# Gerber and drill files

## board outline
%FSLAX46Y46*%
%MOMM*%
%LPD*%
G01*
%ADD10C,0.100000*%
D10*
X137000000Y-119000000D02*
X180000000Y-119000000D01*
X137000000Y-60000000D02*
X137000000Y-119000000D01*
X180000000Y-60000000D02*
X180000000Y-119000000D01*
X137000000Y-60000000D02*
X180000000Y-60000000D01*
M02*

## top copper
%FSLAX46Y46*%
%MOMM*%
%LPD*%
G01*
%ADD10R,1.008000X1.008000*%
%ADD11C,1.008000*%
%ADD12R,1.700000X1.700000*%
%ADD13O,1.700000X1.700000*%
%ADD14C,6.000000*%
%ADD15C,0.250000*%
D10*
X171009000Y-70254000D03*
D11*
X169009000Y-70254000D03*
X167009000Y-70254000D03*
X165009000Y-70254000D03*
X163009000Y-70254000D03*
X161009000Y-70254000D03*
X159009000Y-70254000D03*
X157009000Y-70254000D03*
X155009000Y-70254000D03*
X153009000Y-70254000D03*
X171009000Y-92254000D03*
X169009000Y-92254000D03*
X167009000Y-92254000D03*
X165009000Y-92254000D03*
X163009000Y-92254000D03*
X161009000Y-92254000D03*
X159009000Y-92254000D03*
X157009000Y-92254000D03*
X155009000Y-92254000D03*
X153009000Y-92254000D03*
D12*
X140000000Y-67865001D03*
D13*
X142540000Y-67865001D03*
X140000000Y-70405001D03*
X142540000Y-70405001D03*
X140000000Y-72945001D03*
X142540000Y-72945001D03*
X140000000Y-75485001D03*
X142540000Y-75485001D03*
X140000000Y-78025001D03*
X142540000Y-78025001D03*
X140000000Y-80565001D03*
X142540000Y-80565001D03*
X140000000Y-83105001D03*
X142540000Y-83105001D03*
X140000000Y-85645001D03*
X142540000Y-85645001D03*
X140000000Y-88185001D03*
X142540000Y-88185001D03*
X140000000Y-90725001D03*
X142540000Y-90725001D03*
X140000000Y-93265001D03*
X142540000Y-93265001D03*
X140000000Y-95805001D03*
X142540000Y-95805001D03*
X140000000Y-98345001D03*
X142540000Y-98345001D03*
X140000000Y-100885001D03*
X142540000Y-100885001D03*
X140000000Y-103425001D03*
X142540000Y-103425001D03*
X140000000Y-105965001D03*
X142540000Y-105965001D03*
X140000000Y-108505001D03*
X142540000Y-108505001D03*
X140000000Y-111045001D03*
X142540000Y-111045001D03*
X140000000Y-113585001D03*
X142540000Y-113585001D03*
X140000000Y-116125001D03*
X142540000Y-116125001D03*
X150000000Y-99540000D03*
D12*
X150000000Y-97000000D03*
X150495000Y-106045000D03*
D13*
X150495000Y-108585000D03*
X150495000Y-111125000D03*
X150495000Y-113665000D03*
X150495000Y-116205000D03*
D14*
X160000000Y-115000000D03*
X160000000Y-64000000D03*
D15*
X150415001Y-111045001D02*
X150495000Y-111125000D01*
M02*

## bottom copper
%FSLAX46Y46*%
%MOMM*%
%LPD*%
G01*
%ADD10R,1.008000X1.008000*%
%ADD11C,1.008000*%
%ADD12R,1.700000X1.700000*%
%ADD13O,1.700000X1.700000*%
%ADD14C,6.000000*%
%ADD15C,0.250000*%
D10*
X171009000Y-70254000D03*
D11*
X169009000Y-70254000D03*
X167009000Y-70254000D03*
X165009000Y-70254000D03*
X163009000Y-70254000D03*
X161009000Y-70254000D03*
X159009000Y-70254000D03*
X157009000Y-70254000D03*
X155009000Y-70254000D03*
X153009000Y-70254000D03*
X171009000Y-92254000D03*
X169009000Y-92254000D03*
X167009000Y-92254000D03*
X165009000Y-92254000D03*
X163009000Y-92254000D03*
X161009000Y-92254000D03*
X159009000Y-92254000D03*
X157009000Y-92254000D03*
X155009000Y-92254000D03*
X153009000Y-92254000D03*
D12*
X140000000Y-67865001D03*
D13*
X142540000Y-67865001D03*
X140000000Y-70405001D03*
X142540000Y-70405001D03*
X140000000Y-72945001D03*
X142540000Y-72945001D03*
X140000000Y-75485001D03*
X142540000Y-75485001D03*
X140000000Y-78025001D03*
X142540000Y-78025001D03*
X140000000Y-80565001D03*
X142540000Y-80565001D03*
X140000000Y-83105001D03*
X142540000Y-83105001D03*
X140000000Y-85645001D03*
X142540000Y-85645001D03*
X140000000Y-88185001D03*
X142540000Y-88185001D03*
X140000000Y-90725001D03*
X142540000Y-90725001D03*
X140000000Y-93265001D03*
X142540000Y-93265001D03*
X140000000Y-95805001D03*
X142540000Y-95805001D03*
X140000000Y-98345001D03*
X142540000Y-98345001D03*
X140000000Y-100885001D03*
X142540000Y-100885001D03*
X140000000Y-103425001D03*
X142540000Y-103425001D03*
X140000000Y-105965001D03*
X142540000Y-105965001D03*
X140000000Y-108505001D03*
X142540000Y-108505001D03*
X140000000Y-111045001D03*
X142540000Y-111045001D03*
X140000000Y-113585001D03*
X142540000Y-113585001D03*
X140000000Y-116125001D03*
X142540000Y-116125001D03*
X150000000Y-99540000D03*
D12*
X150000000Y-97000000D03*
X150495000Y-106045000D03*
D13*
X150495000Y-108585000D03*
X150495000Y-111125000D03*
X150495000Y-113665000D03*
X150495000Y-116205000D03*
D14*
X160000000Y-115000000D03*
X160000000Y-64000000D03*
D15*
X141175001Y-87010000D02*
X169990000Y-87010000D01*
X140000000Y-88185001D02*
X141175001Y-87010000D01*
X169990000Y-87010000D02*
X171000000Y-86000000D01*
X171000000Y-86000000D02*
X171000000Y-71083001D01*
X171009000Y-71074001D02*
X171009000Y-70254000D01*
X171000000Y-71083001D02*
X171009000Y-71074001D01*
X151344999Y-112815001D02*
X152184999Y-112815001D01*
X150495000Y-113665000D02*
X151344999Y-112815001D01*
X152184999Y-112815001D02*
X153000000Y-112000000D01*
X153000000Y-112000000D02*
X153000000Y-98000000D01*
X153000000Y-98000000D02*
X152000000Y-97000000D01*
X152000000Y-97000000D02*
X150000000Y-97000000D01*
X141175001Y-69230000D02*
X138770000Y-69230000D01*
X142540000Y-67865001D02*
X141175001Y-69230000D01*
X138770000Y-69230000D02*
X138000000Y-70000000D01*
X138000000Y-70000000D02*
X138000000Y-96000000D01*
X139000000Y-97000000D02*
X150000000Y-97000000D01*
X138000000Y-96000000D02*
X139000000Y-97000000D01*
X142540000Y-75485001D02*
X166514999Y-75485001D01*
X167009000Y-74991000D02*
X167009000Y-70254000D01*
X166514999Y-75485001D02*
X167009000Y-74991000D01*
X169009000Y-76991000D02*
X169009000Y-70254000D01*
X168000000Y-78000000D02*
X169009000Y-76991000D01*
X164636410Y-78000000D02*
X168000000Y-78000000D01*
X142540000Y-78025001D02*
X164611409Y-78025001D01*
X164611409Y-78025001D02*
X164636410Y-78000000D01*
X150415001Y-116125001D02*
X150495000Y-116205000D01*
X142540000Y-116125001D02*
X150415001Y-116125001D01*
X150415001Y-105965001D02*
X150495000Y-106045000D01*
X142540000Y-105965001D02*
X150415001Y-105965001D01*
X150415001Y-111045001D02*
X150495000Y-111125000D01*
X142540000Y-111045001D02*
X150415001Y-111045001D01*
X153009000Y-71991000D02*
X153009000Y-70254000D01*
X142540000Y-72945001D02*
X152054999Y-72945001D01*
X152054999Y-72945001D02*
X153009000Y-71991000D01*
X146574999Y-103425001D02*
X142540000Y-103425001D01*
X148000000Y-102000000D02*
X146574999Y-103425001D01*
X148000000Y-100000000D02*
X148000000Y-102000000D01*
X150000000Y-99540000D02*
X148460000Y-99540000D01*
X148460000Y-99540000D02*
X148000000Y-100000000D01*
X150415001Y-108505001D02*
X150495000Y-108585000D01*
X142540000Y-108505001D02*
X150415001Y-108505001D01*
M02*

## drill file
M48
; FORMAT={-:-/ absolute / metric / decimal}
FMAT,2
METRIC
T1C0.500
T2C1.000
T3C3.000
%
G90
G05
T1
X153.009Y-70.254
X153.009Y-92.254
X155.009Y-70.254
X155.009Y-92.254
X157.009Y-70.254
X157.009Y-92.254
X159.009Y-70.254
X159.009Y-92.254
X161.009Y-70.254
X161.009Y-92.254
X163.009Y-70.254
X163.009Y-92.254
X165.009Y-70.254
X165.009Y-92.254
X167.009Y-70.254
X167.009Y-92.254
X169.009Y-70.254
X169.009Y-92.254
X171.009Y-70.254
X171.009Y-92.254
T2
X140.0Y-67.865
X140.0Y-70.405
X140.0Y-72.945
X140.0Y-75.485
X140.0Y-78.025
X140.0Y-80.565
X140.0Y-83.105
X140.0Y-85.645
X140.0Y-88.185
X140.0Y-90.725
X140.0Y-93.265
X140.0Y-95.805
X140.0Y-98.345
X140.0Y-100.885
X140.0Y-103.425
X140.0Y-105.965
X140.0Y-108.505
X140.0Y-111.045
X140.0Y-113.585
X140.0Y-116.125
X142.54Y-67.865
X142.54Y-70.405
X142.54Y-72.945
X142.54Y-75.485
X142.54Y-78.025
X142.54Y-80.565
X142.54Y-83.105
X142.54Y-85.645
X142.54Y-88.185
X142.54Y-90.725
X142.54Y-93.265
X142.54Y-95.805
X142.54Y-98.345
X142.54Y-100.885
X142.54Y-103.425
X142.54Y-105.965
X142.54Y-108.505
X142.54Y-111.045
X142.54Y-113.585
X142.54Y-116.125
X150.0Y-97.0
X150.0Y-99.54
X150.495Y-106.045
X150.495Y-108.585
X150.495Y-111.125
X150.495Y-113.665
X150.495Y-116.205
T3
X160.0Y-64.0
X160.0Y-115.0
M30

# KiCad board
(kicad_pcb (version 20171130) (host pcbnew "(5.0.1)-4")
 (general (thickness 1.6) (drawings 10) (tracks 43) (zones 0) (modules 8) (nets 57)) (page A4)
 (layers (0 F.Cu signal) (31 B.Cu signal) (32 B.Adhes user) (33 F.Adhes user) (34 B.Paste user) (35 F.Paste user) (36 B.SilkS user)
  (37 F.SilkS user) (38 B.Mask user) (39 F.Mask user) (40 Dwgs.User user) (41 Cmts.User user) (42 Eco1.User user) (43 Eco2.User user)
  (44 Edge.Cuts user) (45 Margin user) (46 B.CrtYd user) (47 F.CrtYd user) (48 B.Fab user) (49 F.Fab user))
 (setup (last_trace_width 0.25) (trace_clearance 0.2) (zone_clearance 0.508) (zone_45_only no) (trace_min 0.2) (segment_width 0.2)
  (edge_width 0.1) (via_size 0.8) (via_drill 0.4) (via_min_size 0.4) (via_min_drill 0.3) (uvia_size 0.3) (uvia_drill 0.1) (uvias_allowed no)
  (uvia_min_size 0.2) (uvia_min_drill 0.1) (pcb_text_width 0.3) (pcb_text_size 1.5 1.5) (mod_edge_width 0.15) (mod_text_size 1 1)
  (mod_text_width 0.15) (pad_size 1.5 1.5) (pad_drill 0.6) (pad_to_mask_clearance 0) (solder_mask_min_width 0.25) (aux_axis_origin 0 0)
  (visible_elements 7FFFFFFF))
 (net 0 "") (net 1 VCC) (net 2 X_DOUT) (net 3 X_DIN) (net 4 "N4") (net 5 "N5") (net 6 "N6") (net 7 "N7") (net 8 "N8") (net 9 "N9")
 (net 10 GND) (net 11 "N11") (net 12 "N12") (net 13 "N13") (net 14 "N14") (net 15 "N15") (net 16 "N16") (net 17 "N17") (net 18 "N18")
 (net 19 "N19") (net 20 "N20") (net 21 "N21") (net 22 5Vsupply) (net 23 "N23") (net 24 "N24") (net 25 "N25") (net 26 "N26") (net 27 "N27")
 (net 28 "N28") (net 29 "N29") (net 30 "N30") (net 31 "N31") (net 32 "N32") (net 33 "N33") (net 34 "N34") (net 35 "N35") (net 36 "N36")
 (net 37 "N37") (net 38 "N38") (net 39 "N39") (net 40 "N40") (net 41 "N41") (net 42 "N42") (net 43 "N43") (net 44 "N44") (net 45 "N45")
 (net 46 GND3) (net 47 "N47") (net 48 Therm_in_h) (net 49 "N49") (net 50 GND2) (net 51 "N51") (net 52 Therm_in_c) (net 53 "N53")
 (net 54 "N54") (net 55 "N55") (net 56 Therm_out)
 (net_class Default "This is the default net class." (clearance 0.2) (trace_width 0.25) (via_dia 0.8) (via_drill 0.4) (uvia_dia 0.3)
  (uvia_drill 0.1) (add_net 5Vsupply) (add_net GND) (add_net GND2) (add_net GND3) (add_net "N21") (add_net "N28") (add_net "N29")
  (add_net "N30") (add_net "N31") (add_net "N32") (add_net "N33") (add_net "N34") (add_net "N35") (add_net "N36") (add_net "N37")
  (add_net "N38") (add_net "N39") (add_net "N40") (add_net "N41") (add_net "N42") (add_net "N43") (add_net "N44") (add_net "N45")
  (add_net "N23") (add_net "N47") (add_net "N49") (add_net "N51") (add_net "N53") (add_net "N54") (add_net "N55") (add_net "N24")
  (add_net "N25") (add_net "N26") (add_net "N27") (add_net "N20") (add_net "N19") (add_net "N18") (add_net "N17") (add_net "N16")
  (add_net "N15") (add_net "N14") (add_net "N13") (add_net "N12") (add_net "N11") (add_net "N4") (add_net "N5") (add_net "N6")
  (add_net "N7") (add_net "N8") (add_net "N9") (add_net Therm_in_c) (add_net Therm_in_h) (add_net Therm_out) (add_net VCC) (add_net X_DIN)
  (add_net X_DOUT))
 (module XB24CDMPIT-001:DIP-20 (layer F.Cu) (at 145 69 270)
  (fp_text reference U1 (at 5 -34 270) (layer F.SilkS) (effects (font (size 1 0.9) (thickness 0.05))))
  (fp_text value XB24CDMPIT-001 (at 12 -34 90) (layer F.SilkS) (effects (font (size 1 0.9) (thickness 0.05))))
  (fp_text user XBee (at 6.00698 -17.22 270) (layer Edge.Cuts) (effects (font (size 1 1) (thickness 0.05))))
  (pad 1 thru_hole rect (at 1.254 -26.009 270) (size 1.008 1.008) (drill 0.5) (layers *.Cu *.Mask) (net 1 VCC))
  (pad 2 thru_hole circle (at 1.254 -24.009 270) (size 1.008 1.008) (drill 0.5) (layers *.Cu *.Mask) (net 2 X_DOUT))
  (pad 3 thru_hole circle (at 1.254 -22.009 270) (size 1.008 1.008) (drill 0.5) (layers *.Cu *.Mask) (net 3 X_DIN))
  (pad 4 thru_hole circle (at 1.254 -20.009 270) (size 1.008 1.008) (drill 0.5) (layers *.Cu *.Mask) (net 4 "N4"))
  (pad 5 thru_hole circle (at 1.254 -18.009 270) (size 1.008 1.008) (drill 0.5) (layers *.Cu *.Mask) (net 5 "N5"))
  (pad 6 thru_hole circle (at 1.254 -16.009 270) (size 1.008 1.008) (drill 0.5) (layers *.Cu *.Mask) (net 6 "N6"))
  (pad 7 thru_hole circle (at 1.254 -14.009 270) (size 1.008 1.008) (drill 0.5) (layers *.Cu *.Mask) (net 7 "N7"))
  (pad 8 thru_hole circle (at 1.254 -12.009 270) (size 1.008 1.008) (drill 0.5) (layers *.Cu *.Mask) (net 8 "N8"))
  (pad 9 thru_hole circle (at 1.254 -10.009 270) (size 1.008 1.008) (drill 0.5) (layers *.Cu *.Mask) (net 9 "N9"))
  (pad 10 thru_hole circle (at 1.254 -8.009 270) (size 1.008 1.008) (drill 0.5) (layers *.Cu *.Mask) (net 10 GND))
  (pad 20 thru_hole circle (at 23.254 -26.009 270) (size 1.008 1.008) (drill 0.5) (layers *.Cu *.Mask) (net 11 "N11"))
  (pad 19 thru_hole circle (at 23.254 -24.009 270) (size 1.008 1.008) (drill 0.5) (layers *.Cu *.Mask) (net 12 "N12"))
  (pad 18 thru_hole circle (at 23.254 -22.009 270) (size 1.008 1.008) (drill 0.5) (layers *.Cu *.Mask) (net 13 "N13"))
  (pad 17 thru_hole circle (at 23.254 -20.009 270) (size 1.008 1.008) (drill 0.5) (layers *.Cu *.Mask) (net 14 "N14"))
  (pad 16 thru_hole circle (at 23.254 -18.009 270) (size 1.008 1.008) (drill 0.5) (layers *.Cu *.Mask) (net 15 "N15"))
  (pad 15 thru_hole circle (at 23.254 -16.009 270) (size 1.008 1.008) (drill 0.5) (layers *.Cu *.Mask) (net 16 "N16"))
  (pad 14 thru_hole circle (at 23.254 -14.009 270) (size 1.008 1.008) (drill 0.5) (layers *.Cu *.Mask) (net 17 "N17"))
  (pad 13 thru_hole circle (at 23.254 -12.009 270) (size 1.008 1.008) (drill 0.5) (layers *.Cu *.Mask) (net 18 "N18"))
  (pad 12 thru_hole circle (at 23.254 -10.009 270) (size 1.008 1.008) (drill 0.5) (layers *.Cu *.Mask) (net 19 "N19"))
  (pad 11 thru_hole circle (at 23.254 -8.009 270) (size 1.008 1.008) (drill 0.5) (layers *.Cu *.Mask) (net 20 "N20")))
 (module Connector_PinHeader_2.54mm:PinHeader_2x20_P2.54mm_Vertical (layer F.Cu) (at 140 67.865001)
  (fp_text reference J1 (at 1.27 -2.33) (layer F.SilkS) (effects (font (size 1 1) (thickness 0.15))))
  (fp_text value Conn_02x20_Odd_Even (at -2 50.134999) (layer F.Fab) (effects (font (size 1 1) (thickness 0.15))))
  (pad 1 thru_hole rect (at 0 0) (size 1.7 1.7) (drill 1) (layers *.Cu *.Mask) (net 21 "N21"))
  (pad 2 thru_hole oval (at 2.54 0) (size 1.7 1.7) (drill 1) (layers *.Cu *.Mask) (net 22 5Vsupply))
  (pad 3 thru_hole oval (at 0 2.54) (size 1.7 1.7) (drill 1) (layers *.Cu *.Mask) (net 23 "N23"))
  (pad 4 thru_hole oval (at 2.54 2.54) (size 1.7 1.7) (drill 1) (layers *.Cu *.Mask) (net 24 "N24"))
  (pad 5 thru_hole oval (at 0 5.08) (size 1.7 1.7) (drill 1) (layers *.Cu *.Mask) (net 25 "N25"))
  (pad 6 thru_hole oval (at 2.54 5.08) (size 1.7 1.7) (drill 1) (layers *.Cu *.Mask) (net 10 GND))
  (pad 7 thru_hole oval (at 0 7.62) (size 1.7 1.7) (drill 1) (layers *.Cu *.Mask) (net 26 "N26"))
  (pad 8 thru_hole oval (at 2.54 7.62) (size 1.7 1.7) (drill 1) (layers *.Cu *.Mask) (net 3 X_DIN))
  (pad 9 thru_hole oval (at 0 10.16) (size 1.7 1.7) (drill 1) (layers *.Cu *.Mask) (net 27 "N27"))
  (pad 10 thru_hole oval (at 2.54 10.16) (size 1.7 1.7) (drill 1) (layers *.Cu *.Mask) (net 2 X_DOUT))
  (pad 11 thru_hole oval (at 0 12.7) (size 1.7 1.7) (drill 1) (layers *.Cu *.Mask) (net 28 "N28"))
  (pad 12 thru_hole oval (at 2.54 12.7) (size 1.7 1.7) (drill 1) (layers *.Cu *.Mask) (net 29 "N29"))
  (pad 13 thru_hole oval (at 0 15.24) (size 1.7 1.7) (drill 1) (layers *.Cu *.Mask) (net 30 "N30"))
  (pad 14 thru_hole oval (at 2.54 15.24) (size 1.7 1.7) (drill 1) (layers *.Cu *.Mask) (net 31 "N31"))
  (pad 15 thru_hole oval (at 0 17.78) (size 1.7 1.7) (drill 1) (layers *.Cu *.Mask) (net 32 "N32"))
  (pad 16 thru_hole oval (at 2.54 17.78) (size 1.7 1.7) (drill 1) (layers *.Cu *.Mask) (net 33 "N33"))
  (pad 17 thru_hole oval (at 0 20.32) (size 1.7 1.7) (drill 1) (layers *.Cu *.Mask) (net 1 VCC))
  (pad 18 thru_hole oval (at 2.54 20.32) (size 1.7 1.7) (drill 1) (layers *.Cu *.Mask) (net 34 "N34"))
  (pad 19 thru_hole oval (at 0 22.86) (size 1.7 1.7) (drill 1) (layers *.Cu *.Mask) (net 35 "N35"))
  (pad 20 thru_hole oval (at 2.54 22.86) (size 1.7 1.7) (drill 1) (layers *.Cu *.Mask) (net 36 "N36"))
  (pad 21 thru_hole oval (at 0 25.4) (size 1.7 1.7) (drill 1) (layers *.Cu *.Mask) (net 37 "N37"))
  (pad 22 thru_hole oval (at 2.54 25.4) (size 1.7 1.7) (drill 1) (layers *.Cu *.Mask) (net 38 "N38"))
  (pad 23 thru_hole oval (at 0 27.94) (size 1.7 1.7) (drill 1) (layers *.Cu *.Mask) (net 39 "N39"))
  (pad 24 thru_hole oval (at 2.54 27.94) (size 1.7 1.7) (drill 1) (layers *.Cu *.Mask) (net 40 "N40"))
  (pad 25 thru_hole oval (at 0 30.48) (size 1.7 1.7) (drill 1) (layers *.Cu *.Mask) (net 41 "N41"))
  (pad 26 thru_hole oval (at 2.54 30.48) (size 1.7 1.7) (drill 1) (layers *.Cu *.Mask) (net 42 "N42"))
  (pad 27 thru_hole oval (at 0 33.02) (size 1.7 1.7) (drill 1) (layers *.Cu *.Mask) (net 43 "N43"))
  (pad 28 thru_hole oval (at 2.54 33.02) (size 1.7 1.7) (drill 1) (layers *.Cu *.Mask) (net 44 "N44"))
  (pad 29 thru_hole oval (at 0 35.56) (size 1.7 1.7) (drill 1) (layers *.Cu *.Mask) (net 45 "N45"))
  (pad 30 thru_hole oval (at 2.54 35.56) (size 1.7 1.7) (drill 1) (layers *.Cu *.Mask) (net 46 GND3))
  (pad 31 thru_hole oval (at 0 38.1) (size 1.7 1.7) (drill 1) (layers *.Cu *.Mask) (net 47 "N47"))
  (pad 32 thru_hole oval (at 2.54 38.1) (size 1.7 1.7) (drill 1) (layers *.Cu *.Mask) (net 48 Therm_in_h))
  (pad 33 thru_hole oval (at 0 40.64) (size 1.7 1.7) (drill 1) (layers *.Cu *.Mask) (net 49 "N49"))
  (pad 34 thru_hole oval (at 2.54 40.64) (size 1.7 1.7) (drill 1) (layers *.Cu *.Mask) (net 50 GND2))
  (pad 35 thru_hole oval (at 0 43.18) (size 1.7 1.7) (drill 1) (layers *.Cu *.Mask) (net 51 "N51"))
  (pad 36 thru_hole oval (at 2.54 43.18) (size 1.7 1.7) (drill 1) (layers *.Cu *.Mask) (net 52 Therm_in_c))
  (pad 37 thru_hole oval (at 0 45.72) (size 1.7 1.7) (drill 1) (layers *.Cu *.Mask) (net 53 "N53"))
  (pad 38 thru_hole oval (at 2.54 45.72) (size 1.7 1.7) (drill 1) (layers *.Cu *.Mask) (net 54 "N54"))
  (pad 39 thru_hole oval (at 0 48.26) (size 1.7 1.7) (drill 1) (layers *.Cu *.Mask) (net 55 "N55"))
  (pad 40 thru_hole oval (at 2.54 48.26) (size 1.7 1.7) (drill 1) (layers *.Cu *.Mask) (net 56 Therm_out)))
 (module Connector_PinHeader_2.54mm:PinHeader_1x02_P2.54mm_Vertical (layer F.Cu) (at 150 97)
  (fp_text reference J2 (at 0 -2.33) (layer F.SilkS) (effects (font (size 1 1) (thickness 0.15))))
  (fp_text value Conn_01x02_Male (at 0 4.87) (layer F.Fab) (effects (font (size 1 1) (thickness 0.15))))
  (pad 2 thru_hole oval (at 0 2.54) (size 1.7 1.7) (drill 1) (layers *.Cu *.Mask) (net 46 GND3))
  (pad 1 thru_hole rect (at 0 0) (size 1.7 1.7) (drill 1) (layers *.Cu *.Mask) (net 22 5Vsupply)))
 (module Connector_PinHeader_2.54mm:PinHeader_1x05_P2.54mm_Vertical (layer F.Cu) (at 150.495 106.045)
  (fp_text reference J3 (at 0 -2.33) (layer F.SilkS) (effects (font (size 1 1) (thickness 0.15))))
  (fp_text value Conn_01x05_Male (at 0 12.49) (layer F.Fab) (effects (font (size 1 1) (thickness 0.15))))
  (pad 1 thru_hole rect (at 0 0) (size 1.7 1.7) (drill 1) (layers *.Cu *.Mask) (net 48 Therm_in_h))
  (pad 2 thru_hole oval (at 0 2.54) (size 1.7 1.7) (drill 1) (layers *.Cu *.Mask) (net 50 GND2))
  (pad 3 thru_hole oval (at 0 5.08) (size 1.7 1.7) (drill 1) (layers *.Cu *.Mask) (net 52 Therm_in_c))
  (pad 4 thru_hole oval (at 0 7.62) (size 1.7 1.7) (drill 1) (layers *.Cu *.Mask) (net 22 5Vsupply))
  (pad 5 thru_hole oval (at 0 10.16) (size 1.7 1.7) (drill 1) (layers *.Cu *.Mask) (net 56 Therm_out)))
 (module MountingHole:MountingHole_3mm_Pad (layer F.Cu) (at 160 115)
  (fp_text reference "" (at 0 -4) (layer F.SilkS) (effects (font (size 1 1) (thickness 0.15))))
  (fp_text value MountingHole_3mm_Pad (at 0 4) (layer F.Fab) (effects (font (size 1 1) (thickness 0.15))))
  (pad 1 thru_hole circle (at 0 0) (size 6 6) (drill 3) (layers *.Cu *.Mask)))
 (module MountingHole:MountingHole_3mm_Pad (layer F.Cu) (at 160 64)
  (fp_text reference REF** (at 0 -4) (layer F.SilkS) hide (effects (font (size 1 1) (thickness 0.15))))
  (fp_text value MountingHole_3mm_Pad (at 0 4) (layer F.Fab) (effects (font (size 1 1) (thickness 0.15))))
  (pad 1 thru_hole circle (at 0 0) (size 6 6) (drill 3) (layers *.Cu *.Mask)))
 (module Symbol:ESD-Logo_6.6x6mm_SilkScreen (layer F.Cu) (at 175 114)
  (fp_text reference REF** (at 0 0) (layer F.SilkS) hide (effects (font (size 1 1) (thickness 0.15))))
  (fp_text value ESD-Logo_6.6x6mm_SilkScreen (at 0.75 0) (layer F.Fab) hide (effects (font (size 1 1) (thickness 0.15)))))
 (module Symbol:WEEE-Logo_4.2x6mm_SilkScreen (layer F.Cu) (at 168 114)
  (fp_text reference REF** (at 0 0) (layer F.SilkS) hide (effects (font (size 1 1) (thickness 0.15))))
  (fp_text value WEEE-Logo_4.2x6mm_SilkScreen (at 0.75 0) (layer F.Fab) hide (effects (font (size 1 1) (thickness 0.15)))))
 (gr_line (start 137 119) (end 180 119) (layer Edge.Cuts) (width 0.1))
 (gr_line (start 137 60) (end 137 119) (layer Edge.Cuts) (width 0.1))
 (gr_line (start 180 60) (end 180 119) (layer Edge.Cuts) (width 0.1))
 (gr_line (start 137 60) (end 180 60) (layer Edge.Cuts) (width 0.1))
 (segment (start 141.175001 87.01) (end 169.99 87.01) (width 0.25) (layer B.Cu) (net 1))
 (segment (start 140 88.185001) (end 141.175001 87.01) (width 0.25) (layer B.Cu) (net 1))
 (segment (start 169.99 87.01) (end 171 86) (width 0.25) (layer B.Cu) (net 1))
 (segment (start 171 86) (end 171 71.083001) (width 0.25) (layer B.Cu) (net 1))
 (segment (start 171.009 71.074001) (end 171.009 70.254) (width 0.25) (layer B.Cu) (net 1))
 (segment (start 171 71.083001) (end 171.009 71.074001) (width 0.25) (layer B.Cu) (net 1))
 (segment (start 151.344999 112.815001) (end 152.184999 112.815001) (width 0.25) (layer B.Cu) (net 22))
 (segment (start 150.495 113.665) (end 151.344999 112.815001) (width 0.25) (layer B.Cu) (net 22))
 (segment (start 152.184999 112.815001) (end 153 112) (width 0.25) (layer B.Cu) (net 22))
 (segment (start 153 112) (end 153 98) (width 0.25) (layer B.Cu) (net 22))
 (segment (start 153 98) (end 152 97) (width 0.25) (layer B.Cu) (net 22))
 (segment (start 152 97) (end 150 97) (width 0.25) (layer B.Cu) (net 22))
 (segment (start 141.175001 69.23) (end 138.77 69.23) (width 0.25) (layer B.Cu) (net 22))
 (segment (start 142.54 67.865001) (end 141.175001 69.23) (width 0.25) (layer B.Cu) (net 22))
 (segment (start 138.77 69.23) (end 138 70) (width 0.25) (layer B.Cu) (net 22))
 (segment (start 138 70) (end 138 96) (width 0.25) (layer B.Cu) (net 22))
 (segment (start 139 97) (end 150 97) (width 0.25) (layer B.Cu) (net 22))
 (segment (start 138 96) (end 139 97) (width 0.25) (layer B.Cu) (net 22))
 (segment (start 142.54 75.485001) (end 166.514999 75.485001) (width 0.25) (layer B.Cu) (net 3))
 (segment (start 167.009 74.991) (end 167.009 70.254) (width 0.25) (layer B.Cu) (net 3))
 (segment (start 166.514999 75.485001) (end 167.009 74.991) (width 0.25) (layer B.Cu) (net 3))
 (segment (start 169.009 76.991) (end 169.009 70.254) (width 0.25) (layer B.Cu) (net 2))
 (segment (start 168 78) (end 169.009 76.991) (width 0.25) (layer B.Cu) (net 2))
 (segment (start 164.63641 78) (end 168 78) (width 0.25) (layer B.Cu) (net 2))
 (segment (start 142.54 78.025001) (end 164.611409 78.025001) (width 0.25) (layer B.Cu) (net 2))
 (segment (start 164.611409 78.025001) (end 164.63641 78) (width 0.25) (layer B.Cu) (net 2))
 (segment (start 150.415001 116.125001) (end 150.495 116.205) (width 0.25) (layer B.Cu) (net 56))
 (segment (start 142.54 116.125001) (end 150.415001 116.125001) (width 0.25) (layer B.Cu) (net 56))
 (segment (start 150.415001 105.965001) (end 150.495 106.045) (width 0.25) (layer B.Cu) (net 48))
 (segment (start 142.54 105.965001) (end 150.415001 105.965001) (width 0.25) (layer B.Cu) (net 48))
 (segment (start 150.415001 111.045001) (end 150.495 111.125) (width 0.25) (layer F.Cu) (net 52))
 (segment (start 150.415001 111.045001) (end 150.495 111.125) (width 0.25) (layer B.Cu) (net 52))
 (segment (start 142.54 111.045001) (end 150.415001 111.045001) (width 0.25) (layer B.Cu) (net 52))
 (segment (start 153.009 71.991) (end 153.009 70.254) (width 0.25) (layer B.Cu) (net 10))
 (segment (start 142.54 72.945001) (end 152.054999 72.945001) (width 0.25) (layer B.Cu) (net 10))
 (segment (start 152.054999 72.945001) (end 153.009 71.991) (width 0.25) (layer B.Cu) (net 10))
 (segment (start 146.574999 103.425001) (end 142.54 103.425001) (width 0.25) (layer B.Cu) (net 46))
 (segment (start 148 102) (end 146.574999 103.425001) (width 0.25) (layer B.Cu) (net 46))
 (segment (start 148 100) (end 148 102) (width 0.25) (layer B.Cu) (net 46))
 (segment (start 150 99.54) (end 148.46 99.54) (width 0.25) (layer B.Cu) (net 46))
 (segment (start 148.46 99.54) (end 148 100) (width 0.25) (layer B.Cu) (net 46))
 (segment (start 150.415001 108.505001) (end 150.495 108.585) (width 0.25) (layer B.Cu) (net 50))
 (segment (start 142.54 108.505001) (end 150.415001 108.505001) (width 0.25) (layer B.Cu) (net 50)))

